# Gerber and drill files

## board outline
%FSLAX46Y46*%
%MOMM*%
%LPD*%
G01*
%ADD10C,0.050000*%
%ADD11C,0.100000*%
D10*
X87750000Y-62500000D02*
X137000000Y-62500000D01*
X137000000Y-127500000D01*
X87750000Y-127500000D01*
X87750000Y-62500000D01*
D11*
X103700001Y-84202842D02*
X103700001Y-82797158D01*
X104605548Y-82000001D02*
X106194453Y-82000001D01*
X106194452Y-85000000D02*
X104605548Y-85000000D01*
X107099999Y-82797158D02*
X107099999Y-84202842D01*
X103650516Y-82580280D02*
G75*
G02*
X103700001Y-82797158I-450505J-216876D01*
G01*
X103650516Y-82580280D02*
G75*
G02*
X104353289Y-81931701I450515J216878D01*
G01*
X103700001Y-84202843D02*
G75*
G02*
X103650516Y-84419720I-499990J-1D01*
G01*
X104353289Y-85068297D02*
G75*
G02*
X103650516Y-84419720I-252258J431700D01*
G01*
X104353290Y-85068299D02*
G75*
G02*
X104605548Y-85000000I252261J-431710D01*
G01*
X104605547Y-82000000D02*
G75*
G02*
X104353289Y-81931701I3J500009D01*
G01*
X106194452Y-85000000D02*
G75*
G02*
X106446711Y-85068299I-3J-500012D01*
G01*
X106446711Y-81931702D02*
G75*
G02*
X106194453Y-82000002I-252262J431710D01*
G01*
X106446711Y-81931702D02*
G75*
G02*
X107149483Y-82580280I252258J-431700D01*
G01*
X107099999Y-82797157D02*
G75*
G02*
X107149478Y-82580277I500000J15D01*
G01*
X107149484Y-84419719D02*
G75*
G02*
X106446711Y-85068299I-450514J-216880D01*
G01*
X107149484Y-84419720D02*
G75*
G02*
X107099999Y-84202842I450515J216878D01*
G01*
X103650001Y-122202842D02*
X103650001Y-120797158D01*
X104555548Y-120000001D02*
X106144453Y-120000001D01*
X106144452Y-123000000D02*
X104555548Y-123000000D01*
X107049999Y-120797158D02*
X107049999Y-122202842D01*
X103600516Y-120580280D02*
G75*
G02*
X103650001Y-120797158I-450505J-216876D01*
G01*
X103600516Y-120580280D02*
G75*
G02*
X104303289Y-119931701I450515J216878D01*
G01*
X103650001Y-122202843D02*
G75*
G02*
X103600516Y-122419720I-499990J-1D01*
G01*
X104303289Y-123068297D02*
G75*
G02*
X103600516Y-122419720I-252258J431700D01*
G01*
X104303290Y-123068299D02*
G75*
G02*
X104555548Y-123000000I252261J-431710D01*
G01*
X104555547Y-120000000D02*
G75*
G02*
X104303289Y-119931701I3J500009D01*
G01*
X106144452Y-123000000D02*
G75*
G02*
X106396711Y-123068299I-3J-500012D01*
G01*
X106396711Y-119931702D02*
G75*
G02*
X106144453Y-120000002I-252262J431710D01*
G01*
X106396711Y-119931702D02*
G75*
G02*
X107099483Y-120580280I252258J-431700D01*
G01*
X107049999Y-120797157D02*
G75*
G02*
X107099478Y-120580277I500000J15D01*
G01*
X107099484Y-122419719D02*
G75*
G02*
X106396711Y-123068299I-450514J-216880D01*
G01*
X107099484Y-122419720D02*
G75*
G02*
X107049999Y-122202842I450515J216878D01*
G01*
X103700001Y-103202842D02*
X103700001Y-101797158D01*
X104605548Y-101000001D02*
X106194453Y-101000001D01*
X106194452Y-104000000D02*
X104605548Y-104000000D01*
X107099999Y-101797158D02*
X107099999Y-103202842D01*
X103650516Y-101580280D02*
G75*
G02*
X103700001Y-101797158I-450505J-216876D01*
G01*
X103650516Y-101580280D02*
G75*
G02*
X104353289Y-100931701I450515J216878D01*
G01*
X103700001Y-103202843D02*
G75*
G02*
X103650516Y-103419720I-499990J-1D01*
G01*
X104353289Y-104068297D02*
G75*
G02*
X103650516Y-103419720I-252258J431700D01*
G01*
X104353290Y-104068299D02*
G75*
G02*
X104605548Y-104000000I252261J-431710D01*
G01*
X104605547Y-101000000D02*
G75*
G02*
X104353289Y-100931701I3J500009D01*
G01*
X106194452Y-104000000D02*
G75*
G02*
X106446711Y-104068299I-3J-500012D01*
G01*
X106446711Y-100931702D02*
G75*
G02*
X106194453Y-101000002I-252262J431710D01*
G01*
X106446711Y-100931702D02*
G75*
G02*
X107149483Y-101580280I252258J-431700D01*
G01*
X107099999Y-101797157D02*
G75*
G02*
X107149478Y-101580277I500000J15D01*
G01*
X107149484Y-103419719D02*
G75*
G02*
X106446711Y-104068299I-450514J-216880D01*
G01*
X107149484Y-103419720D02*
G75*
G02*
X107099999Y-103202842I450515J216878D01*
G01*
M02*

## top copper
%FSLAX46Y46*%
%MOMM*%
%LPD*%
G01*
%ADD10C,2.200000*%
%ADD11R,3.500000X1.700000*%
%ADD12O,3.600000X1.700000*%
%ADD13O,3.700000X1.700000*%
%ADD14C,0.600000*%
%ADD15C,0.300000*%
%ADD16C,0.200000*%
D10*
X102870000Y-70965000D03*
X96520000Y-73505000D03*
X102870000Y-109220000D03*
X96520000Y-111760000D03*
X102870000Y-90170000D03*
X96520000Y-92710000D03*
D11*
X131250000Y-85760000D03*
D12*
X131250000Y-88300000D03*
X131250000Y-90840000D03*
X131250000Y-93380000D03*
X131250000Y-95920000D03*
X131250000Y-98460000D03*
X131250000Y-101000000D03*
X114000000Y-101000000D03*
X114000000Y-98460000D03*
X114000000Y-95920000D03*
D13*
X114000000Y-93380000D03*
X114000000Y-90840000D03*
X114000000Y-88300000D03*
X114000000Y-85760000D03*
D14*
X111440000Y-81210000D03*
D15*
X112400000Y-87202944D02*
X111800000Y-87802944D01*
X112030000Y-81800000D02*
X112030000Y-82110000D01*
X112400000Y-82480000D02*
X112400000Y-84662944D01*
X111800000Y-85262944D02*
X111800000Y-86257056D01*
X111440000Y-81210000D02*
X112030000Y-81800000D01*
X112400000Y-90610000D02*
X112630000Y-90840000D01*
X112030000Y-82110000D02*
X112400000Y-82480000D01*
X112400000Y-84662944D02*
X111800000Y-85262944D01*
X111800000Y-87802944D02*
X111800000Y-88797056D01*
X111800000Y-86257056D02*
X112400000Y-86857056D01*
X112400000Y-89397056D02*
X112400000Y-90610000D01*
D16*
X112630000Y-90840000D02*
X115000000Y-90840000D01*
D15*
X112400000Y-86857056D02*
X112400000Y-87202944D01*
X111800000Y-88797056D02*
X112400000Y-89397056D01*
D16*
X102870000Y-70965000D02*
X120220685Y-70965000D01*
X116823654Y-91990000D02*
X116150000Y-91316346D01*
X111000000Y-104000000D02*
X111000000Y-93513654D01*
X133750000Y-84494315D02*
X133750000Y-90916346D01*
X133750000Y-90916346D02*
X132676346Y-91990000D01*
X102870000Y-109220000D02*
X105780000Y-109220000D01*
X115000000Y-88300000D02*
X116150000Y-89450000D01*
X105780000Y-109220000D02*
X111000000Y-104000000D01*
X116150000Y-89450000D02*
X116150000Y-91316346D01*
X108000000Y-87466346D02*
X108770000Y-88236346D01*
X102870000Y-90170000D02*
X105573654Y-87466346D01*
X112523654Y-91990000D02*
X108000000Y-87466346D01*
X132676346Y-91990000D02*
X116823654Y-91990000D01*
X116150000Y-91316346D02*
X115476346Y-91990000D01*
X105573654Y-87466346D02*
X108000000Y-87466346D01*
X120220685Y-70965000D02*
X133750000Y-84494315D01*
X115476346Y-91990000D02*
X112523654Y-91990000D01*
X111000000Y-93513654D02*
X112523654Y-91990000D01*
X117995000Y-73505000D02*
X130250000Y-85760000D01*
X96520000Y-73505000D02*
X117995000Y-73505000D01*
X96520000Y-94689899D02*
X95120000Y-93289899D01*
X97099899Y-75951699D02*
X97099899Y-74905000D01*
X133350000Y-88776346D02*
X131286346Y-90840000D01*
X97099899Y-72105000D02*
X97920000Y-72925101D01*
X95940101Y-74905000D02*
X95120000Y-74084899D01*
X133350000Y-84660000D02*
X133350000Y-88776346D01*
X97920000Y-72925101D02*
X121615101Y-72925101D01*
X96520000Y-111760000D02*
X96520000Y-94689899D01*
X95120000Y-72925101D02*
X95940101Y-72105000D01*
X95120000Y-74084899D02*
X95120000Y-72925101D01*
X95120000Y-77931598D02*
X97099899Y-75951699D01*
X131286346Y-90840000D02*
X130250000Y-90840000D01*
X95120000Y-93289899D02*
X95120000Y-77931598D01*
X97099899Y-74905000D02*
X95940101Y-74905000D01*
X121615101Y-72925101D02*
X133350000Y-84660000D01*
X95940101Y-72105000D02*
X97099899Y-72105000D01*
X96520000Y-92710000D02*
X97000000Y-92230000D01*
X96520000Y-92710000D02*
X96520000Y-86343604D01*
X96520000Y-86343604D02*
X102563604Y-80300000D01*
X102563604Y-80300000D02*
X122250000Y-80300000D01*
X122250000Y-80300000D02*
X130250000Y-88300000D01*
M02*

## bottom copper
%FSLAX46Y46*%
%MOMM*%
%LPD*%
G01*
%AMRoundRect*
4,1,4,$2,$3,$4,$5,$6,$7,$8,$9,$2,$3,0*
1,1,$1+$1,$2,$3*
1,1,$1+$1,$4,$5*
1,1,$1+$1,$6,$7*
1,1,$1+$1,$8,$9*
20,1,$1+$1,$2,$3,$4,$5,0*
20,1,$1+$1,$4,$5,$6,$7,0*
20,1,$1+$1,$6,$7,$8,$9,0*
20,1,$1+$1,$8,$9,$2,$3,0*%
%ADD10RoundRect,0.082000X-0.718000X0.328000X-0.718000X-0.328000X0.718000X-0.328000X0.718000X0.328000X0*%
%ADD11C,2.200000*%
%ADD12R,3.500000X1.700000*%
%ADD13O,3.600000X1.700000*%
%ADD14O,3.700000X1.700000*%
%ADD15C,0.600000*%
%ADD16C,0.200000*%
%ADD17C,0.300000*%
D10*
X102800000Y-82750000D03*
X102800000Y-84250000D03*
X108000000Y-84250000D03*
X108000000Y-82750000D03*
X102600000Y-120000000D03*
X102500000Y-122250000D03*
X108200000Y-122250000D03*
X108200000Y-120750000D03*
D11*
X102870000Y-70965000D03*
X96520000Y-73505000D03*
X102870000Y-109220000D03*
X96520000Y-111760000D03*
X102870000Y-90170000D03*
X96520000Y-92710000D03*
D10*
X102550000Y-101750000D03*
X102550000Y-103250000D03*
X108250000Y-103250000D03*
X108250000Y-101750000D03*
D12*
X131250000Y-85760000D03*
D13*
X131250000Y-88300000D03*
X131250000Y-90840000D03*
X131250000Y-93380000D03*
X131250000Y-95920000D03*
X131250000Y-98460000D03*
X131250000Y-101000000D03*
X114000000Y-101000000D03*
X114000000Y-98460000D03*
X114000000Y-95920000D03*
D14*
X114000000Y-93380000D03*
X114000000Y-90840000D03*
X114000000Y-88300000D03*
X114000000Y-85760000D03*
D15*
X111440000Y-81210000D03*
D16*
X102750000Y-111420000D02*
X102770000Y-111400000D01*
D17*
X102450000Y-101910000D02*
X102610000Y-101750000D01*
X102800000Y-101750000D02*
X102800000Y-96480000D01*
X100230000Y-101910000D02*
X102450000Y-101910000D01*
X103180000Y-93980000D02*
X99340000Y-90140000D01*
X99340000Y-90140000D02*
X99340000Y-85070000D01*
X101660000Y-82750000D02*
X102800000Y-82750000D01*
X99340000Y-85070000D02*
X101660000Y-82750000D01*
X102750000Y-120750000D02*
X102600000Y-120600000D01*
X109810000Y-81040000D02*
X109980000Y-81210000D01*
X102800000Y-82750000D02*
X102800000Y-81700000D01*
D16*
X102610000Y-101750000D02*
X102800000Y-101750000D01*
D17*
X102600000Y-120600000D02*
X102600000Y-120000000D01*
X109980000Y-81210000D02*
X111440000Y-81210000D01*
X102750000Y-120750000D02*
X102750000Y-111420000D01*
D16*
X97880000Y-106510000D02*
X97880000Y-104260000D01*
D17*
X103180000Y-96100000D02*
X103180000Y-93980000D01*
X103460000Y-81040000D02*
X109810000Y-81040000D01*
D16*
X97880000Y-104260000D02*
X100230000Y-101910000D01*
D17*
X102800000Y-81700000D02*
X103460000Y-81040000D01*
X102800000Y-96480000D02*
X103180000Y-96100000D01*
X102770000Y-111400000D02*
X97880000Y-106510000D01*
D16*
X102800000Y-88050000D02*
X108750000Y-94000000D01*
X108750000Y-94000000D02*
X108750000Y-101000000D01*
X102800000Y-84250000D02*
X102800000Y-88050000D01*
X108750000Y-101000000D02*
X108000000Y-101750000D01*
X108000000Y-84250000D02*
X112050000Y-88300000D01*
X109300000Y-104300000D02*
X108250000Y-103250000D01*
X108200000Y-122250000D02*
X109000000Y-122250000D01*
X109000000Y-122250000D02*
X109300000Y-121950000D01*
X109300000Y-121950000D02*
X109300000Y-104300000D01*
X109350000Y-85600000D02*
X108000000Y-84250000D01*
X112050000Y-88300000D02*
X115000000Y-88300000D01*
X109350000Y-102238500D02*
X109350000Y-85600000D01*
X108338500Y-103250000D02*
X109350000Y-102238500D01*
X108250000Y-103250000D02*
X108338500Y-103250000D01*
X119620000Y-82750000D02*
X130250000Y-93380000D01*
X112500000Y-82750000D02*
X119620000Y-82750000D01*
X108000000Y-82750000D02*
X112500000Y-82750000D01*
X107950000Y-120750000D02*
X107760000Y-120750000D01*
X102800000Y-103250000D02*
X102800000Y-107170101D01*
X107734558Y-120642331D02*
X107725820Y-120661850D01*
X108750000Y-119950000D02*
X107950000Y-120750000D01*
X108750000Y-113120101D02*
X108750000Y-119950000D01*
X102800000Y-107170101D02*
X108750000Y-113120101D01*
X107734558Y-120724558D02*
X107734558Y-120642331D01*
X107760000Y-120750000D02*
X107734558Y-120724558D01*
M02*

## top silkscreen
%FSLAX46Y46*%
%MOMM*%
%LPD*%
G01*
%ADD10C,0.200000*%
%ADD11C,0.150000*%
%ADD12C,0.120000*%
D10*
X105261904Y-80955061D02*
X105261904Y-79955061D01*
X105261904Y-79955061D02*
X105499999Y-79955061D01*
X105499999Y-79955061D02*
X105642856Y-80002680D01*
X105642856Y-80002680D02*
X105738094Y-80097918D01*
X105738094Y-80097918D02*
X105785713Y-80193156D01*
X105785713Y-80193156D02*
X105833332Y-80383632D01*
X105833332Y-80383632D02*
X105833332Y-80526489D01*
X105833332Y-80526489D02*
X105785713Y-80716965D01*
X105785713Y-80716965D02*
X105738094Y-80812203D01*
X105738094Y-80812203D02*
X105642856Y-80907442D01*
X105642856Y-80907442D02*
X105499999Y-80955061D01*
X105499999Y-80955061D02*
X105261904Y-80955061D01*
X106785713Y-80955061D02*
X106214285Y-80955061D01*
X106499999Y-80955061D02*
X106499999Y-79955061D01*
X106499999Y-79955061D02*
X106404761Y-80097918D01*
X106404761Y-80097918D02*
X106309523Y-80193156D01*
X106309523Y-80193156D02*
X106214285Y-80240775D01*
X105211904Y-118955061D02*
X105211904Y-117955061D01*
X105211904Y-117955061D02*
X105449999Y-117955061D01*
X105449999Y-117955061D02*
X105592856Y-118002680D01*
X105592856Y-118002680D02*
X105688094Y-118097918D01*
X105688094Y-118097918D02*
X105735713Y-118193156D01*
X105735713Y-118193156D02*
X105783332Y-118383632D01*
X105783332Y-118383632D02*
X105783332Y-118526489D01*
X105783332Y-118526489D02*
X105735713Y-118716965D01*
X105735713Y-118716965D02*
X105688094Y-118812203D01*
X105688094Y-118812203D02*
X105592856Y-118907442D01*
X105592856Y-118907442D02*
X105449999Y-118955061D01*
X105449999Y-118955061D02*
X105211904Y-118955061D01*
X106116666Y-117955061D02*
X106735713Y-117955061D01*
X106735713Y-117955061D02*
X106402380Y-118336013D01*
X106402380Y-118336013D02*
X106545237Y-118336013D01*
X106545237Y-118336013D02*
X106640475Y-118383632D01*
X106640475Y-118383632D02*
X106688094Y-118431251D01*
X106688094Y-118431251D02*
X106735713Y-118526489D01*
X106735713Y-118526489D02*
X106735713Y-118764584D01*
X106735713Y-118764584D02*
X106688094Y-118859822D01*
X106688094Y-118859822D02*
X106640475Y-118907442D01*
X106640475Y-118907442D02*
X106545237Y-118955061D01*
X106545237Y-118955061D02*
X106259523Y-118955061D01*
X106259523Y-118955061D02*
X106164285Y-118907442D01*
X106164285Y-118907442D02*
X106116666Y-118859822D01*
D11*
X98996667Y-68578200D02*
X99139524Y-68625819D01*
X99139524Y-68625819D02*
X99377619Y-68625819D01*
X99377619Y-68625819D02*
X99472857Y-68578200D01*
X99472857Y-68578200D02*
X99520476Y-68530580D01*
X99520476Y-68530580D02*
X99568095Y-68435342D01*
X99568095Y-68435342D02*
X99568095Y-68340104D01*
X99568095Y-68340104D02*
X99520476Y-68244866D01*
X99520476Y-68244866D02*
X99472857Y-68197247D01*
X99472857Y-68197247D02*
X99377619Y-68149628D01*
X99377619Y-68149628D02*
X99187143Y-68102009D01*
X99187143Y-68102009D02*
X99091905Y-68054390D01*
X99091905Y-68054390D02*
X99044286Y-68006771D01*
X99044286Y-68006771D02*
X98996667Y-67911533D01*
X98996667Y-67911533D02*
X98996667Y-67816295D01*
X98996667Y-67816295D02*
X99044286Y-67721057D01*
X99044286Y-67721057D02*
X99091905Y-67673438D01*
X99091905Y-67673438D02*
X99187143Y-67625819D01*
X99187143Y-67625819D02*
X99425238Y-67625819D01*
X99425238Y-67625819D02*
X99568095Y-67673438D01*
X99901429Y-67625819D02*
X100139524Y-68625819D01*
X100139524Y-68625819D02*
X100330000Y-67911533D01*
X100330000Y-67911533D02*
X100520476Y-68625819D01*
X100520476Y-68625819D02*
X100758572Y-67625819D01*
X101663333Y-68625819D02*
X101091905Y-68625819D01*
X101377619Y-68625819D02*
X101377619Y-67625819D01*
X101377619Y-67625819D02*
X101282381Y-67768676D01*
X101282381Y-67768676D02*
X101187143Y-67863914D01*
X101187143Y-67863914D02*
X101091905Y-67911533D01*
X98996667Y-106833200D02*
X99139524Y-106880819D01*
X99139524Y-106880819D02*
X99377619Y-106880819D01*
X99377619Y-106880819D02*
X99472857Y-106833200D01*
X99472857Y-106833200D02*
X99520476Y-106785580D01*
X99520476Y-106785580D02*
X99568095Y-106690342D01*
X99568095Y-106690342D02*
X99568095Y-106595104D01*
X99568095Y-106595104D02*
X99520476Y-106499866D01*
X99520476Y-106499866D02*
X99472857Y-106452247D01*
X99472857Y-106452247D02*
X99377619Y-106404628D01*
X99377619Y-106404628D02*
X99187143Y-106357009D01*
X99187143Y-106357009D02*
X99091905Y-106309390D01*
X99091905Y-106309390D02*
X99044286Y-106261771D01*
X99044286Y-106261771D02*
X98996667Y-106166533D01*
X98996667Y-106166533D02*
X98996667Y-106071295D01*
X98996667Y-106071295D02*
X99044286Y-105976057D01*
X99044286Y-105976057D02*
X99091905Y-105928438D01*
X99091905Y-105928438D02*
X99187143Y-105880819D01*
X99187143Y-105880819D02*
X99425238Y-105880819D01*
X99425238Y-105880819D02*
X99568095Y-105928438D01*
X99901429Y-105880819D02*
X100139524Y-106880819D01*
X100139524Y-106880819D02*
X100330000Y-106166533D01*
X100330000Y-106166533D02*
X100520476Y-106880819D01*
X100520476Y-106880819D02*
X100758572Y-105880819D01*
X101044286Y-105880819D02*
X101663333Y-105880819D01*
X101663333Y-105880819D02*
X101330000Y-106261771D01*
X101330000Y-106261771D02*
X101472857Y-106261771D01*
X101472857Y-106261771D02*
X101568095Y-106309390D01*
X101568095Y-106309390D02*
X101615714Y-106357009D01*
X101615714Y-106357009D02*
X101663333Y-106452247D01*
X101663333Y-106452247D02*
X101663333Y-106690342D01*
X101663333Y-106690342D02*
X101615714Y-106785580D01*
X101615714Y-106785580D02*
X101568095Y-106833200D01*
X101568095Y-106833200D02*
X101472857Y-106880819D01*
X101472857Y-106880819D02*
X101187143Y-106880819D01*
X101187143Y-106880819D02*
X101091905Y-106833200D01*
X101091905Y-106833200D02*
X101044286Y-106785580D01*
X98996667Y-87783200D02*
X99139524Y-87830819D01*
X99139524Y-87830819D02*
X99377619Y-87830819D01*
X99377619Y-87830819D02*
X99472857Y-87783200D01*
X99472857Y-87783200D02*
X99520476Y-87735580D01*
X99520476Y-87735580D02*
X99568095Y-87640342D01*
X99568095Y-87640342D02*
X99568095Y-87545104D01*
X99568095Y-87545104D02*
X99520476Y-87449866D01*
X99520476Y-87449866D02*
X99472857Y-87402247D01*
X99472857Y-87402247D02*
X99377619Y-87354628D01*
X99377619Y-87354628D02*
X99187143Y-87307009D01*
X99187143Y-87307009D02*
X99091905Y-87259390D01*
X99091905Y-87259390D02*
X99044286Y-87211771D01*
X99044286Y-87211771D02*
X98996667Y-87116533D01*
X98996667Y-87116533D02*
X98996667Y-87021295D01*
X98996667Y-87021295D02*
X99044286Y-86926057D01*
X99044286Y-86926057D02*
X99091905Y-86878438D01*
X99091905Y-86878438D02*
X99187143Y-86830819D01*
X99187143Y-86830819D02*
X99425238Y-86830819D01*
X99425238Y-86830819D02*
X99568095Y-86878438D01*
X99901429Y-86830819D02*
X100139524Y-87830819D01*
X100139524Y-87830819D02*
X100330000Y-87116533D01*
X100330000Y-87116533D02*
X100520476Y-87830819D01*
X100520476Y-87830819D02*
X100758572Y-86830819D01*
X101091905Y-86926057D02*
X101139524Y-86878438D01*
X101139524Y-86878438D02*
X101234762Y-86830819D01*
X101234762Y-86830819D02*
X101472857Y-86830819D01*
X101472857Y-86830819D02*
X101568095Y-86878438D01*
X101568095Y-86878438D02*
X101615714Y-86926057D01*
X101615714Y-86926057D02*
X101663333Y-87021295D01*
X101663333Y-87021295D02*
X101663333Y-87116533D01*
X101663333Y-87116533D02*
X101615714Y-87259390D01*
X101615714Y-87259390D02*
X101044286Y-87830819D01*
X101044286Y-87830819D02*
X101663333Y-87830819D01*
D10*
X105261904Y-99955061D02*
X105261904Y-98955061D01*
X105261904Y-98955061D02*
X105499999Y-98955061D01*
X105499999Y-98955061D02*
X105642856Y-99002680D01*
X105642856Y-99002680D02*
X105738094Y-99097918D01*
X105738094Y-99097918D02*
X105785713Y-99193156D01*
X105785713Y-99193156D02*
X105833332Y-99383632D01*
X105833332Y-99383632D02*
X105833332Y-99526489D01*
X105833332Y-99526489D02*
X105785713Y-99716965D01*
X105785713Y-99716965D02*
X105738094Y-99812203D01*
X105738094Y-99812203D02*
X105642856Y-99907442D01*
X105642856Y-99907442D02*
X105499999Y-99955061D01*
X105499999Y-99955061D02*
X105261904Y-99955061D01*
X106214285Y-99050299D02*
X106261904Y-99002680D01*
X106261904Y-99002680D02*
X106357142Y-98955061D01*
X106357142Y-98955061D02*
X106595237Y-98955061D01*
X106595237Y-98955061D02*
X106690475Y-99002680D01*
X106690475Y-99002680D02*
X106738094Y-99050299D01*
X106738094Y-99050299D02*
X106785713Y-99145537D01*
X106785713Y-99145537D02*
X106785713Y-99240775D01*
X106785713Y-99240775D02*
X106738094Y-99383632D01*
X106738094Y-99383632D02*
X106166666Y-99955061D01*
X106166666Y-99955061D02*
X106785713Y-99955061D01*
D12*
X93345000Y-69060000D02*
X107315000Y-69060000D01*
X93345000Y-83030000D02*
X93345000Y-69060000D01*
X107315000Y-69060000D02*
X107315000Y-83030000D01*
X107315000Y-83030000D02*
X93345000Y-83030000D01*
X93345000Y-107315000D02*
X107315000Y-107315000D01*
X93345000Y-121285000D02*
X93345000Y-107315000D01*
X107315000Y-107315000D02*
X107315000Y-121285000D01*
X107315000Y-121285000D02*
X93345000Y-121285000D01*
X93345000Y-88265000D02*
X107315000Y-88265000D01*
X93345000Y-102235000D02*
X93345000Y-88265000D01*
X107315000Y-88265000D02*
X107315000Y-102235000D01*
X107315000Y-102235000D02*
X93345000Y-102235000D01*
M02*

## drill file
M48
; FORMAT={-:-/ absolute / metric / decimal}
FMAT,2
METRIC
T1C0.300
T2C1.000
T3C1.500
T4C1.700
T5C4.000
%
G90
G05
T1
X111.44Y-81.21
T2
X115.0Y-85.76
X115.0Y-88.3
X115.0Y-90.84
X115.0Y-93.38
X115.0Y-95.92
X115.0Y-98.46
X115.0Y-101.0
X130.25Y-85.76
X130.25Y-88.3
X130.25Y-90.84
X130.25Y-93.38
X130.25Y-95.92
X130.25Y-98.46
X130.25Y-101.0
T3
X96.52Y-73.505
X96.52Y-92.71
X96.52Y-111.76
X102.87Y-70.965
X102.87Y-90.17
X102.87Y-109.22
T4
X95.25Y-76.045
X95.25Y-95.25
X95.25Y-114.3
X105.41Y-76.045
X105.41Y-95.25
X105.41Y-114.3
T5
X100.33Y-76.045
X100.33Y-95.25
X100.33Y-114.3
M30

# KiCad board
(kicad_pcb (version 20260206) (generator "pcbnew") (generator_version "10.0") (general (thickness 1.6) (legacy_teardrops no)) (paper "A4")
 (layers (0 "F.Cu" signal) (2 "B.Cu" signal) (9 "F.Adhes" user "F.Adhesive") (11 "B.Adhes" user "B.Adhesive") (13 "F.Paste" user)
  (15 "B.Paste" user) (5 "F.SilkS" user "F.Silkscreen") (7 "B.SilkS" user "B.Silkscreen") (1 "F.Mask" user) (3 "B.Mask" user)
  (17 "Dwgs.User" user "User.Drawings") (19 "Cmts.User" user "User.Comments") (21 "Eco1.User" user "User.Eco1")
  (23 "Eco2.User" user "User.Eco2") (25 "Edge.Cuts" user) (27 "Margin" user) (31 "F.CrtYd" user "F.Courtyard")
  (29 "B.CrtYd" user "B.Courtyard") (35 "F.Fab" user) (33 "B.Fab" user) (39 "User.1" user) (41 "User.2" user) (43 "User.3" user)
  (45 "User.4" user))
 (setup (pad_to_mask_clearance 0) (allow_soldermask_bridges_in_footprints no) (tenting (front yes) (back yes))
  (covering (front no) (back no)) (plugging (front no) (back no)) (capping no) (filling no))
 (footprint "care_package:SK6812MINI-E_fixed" (layer "F.Cu") (at 105.399999 83.602842)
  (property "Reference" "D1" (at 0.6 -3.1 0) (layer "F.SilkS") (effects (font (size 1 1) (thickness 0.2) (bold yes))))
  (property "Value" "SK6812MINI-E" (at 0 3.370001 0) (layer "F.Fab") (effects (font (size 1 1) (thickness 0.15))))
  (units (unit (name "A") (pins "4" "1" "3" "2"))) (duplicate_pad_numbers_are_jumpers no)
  (fp_line (start -1.699998 0.6) (end -1.699998 -0.805684) (stroke (width 0.1) (type solid)) (layer "Edge.Cuts"))
  (fp_line (start -0.794451 -1.602841) (end 0.794454 -1.602841) (stroke (width 0.1) (type solid)) (layer "Edge.Cuts"))
  (fp_line (start 0.794453 1.397158) (end -0.794451 1.397158) (stroke (width 0.1) (type solid)) (layer "Edge.Cuts"))
  (fp_line (start 1.7 -0.805684) (end 1.7 0.6) (stroke (width 0.1) (type solid)) (layer "Edge.Cuts"))
  (fp_arc (start -1.749483 -1.022562) (mid -1.712526 -0.91691) (end -1.699998 -0.805684) (stroke (width 0.1) (type solid))
   (layer "Edge.Cuts"))
  (fp_arc (start -1.749483 -1.022562) (mid -1.63807 -1.606877) (end -1.04671 -1.671141) (stroke (width 0.1) (type solid))
   (layer "Edge.Cuts"))
  (fp_arc (start -1.699998 0.600001) (mid -1.712526 0.711226) (end -1.749483 0.816878) (stroke (width 0.1) (type solid)) (layer "Edge.Cuts"))
  (fp_arc (start -1.04671 1.465455) (mid -1.638069 1.401192) (end -1.749483 0.816878) (stroke (width 0.1) (type solid)) (layer "Edge.Cuts"))
  (fp_arc (start -1.046709 1.465457) (mid -0.925121 1.414535) (end -0.794451 1.397158) (stroke (width 0.1) (type solid)) (layer "Edge.Cuts"))
  (fp_arc (start -0.794452 -1.602842) (mid -0.925122 -1.620219) (end -1.04671 -1.671141) (stroke (width 0.1) (type solid))
   (layer "Edge.Cuts"))
  (fp_arc (start 0.794453 1.397158) (mid 0.925124 1.414535) (end 1.046712 1.465457) (stroke (width 0.1) (type solid)) (layer "Edge.Cuts"))
  (fp_arc (start 1.046712 -1.67114) (mid 0.925124 -1.620218) (end 0.794454 -1.602841) (stroke (width 0.1) (type solid)) (layer "Edge.Cuts"))
  (fp_arc (start 1.046712 -1.67114) (mid 1.638072 -1.606876) (end 1.749485 -1.022562) (stroke (width 0.1) (type solid)) (layer "Edge.Cuts"))
  (fp_arc (start 1.7 -0.805685) (mid 1.712528 -0.91691) (end 1.749485 -1.022562) (stroke (width 0.1) (type solid)) (layer "Edge.Cuts"))
  (fp_arc (start 1.749485 0.816877) (mid 1.638073 1.401193) (end 1.046712 1.465457) (stroke (width 0.1) (type solid)) (layer "Edge.Cuts"))
  (fp_arc (start 1.749485 0.816878) (mid 1.712528 0.711226) (end 1.7 0.6) (stroke (width 0.1) (type solid)) (layer "Edge.Cuts"))
  (pad "1" smd roundrect (at -2.599999 -0.852842 270) (size 0.82 1.6) (layers "B.Cu" "B.Mask" "B.Paste") (roundrect_rratio 0.1) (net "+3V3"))
  (pad "2" smd roundrect (at -2.599999 0.647158 270) (size 0.82 1.6) (layers "B.Cu" "B.Mask" "B.Paste") (roundrect_rratio 0.1)
   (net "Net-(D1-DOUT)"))
  (pad "3" smd roundrect (at 2.600001 0.647158 270) (size 0.82 1.6) (layers "B.Cu" "B.Mask" "B.Paste") (roundrect_rratio 0.1) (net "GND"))
  (pad "4" smd roundrect (at 2.600001 -0.852842 270) (size 0.82 1.6) (layers "B.Cu" "B.Mask" "B.Paste") (roundrect_rratio 0.1)
   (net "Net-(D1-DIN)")))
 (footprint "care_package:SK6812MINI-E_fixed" (layer "F.Cu") (at 105.349999 121.602842)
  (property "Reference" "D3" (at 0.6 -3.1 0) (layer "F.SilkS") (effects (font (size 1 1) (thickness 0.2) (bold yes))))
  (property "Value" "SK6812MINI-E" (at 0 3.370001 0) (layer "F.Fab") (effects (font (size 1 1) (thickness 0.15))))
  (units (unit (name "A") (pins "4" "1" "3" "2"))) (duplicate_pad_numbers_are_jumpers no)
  (fp_line (start -1.699998 0.6) (end -1.699998 -0.805684) (stroke (width 0.1) (type solid)) (layer "Edge.Cuts"))
  (fp_line (start -0.794451 -1.602841) (end 0.794454 -1.602841) (stroke (width 0.1) (type solid)) (layer "Edge.Cuts"))
  (fp_line (start 0.794453 1.397158) (end -0.794451 1.397158) (stroke (width 0.1) (type solid)) (layer "Edge.Cuts"))
  (fp_line (start 1.7 -0.805684) (end 1.7 0.6) (stroke (width 0.1) (type solid)) (layer "Edge.Cuts"))
  (fp_arc (start -1.749483 -1.022562) (mid -1.712526 -0.91691) (end -1.699998 -0.805684) (stroke (width 0.1) (type solid))
   (layer "Edge.Cuts"))
  (fp_arc (start -1.749483 -1.022562) (mid -1.63807 -1.606877) (end -1.04671 -1.671141) (stroke (width 0.1) (type solid))
   (layer "Edge.Cuts"))
  (fp_arc (start -1.699998 0.600001) (mid -1.712526 0.711226) (end -1.749483 0.816878) (stroke (width 0.1) (type solid)) (layer "Edge.Cuts"))
  (fp_arc (start -1.04671 1.465455) (mid -1.638069 1.401192) (end -1.749483 0.816878) (stroke (width 0.1) (type solid)) (layer "Edge.Cuts"))
  (fp_arc (start -1.046709 1.465457) (mid -0.925121 1.414535) (end -0.794451 1.397158) (stroke (width 0.1) (type solid)) (layer "Edge.Cuts"))
  (fp_arc (start -0.794452 -1.602842) (mid -0.925122 -1.620219) (end -1.04671 -1.671141) (stroke (width 0.1) (type solid))
   (layer "Edge.Cuts"))
  (fp_arc (start 0.794453 1.397158) (mid 0.925124 1.414535) (end 1.046712 1.465457) (stroke (width 0.1) (type solid)) (layer "Edge.Cuts"))
  (fp_arc (start 1.046712 -1.67114) (mid 0.925124 -1.620218) (end 0.794454 -1.602841) (stroke (width 0.1) (type solid)) (layer "Edge.Cuts"))
  (fp_arc (start 1.046712 -1.67114) (mid 1.638072 -1.606876) (end 1.749485 -1.022562) (stroke (width 0.1) (type solid)) (layer "Edge.Cuts"))
  (fp_arc (start 1.7 -0.805685) (mid 1.712528 -0.91691) (end 1.749485 -1.022562) (stroke (width 0.1) (type solid)) (layer "Edge.Cuts"))
  (fp_arc (start 1.749485 0.816877) (mid 1.638073 1.401193) (end 1.046712 1.465457) (stroke (width 0.1) (type solid)) (layer "Edge.Cuts"))
  (fp_arc (start 1.749485 0.816878) (mid 1.712528 0.711226) (end 1.7 0.6) (stroke (width 0.1) (type solid)) (layer "Edge.Cuts"))
  (pad "1" smd roundrect (at -2.749999 -1.602842 270) (size 0.82 1.6) (layers "B.Cu" "B.Mask" "B.Paste") (roundrect_rratio 0.1) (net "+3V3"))
  (pad "2" smd roundrect (at -2.849999 0.647158 270) (size 0.82 1.6) (layers "B.Cu" "B.Mask" "B.Paste") (roundrect_rratio 0.1)
   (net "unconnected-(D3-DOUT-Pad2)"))
  (pad "3" smd roundrect (at 2.850001 0.647158 270) (size 0.82 1.6) (layers "B.Cu" "B.Mask" "B.Paste") (roundrect_rratio 0.1) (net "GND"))
  (pad "4" smd roundrect (at 2.850001 -0.852842 270) (size 0.82 1.6) (layers "B.Cu" "B.Mask" "B.Paste") (roundrect_rratio 0.1)
   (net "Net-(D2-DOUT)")))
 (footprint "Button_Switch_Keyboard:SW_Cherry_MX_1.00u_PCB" (layer "F.Cu") (at 102.87 70.965)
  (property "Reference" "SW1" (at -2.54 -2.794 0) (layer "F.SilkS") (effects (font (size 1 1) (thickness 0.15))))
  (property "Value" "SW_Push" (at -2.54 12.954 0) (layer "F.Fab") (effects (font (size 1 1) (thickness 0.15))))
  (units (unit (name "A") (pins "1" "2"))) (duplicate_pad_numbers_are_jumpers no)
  (fp_line (start -9.525 -1.905) (end 4.445 -1.905) (stroke (width 0.12) (type solid)) (layer "F.SilkS"))
  (fp_line (start -9.525 12.065) (end -9.525 -1.905) (stroke (width 0.12) (type solid)) (layer "F.SilkS"))
  (fp_line (start 4.445 -1.905) (end 4.445 12.065) (stroke (width 0.12) (type solid)) (layer "F.SilkS"))
  (fp_line (start 4.445 12.065) (end -9.525 12.065) (stroke (width 0.12) (type solid)) (layer "F.SilkS"))
  (pad "" np_thru_hole circle (at -7.62 5.08) (size 1.7 1.7) (drill 1.7) (layers "*.Cu" "*.Mask"))
  (pad "" np_thru_hole circle (at -2.54 5.08) (size 4 4) (drill 4) (layers "*.Cu" "*.Mask"))
  (pad "" np_thru_hole circle (at 2.54 5.08) (size 1.7 1.7) (drill 1.7) (layers "*.Cu" "*.Mask"))
  (pad "1" thru_hole circle (at 0 0) (size 2.2 2.2) (drill 1.5) (layers "*.Cu" "*.Mask") (remove_unused_layers no) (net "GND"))
  (pad "2" thru_hole circle (at -6.35 2.54) (size 2.2 2.2) (drill 1.5) (layers "*.Cu" "*.Mask") (remove_unused_layers no)
   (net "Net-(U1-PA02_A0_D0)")))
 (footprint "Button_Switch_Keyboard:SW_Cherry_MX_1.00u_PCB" (layer "F.Cu") (at 102.87 109.22)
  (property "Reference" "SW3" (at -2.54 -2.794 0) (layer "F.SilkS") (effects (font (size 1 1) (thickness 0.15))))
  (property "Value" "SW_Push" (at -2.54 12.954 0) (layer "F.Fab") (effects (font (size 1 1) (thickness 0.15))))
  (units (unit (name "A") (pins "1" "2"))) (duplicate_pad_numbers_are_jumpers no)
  (fp_line (start -9.525 -1.905) (end 4.445 -1.905) (stroke (width 0.12) (type solid)) (layer "F.SilkS"))
  (fp_line (start -9.525 12.065) (end -9.525 -1.905) (stroke (width 0.12) (type solid)) (layer "F.SilkS"))
  (fp_line (start 4.445 -1.905) (end 4.445 12.065) (stroke (width 0.12) (type solid)) (layer "F.SilkS"))
  (fp_line (start 4.445 12.065) (end -9.525 12.065) (stroke (width 0.12) (type solid)) (layer "F.SilkS"))
  (pad "" np_thru_hole circle (at -7.62 5.08) (size 1.7 1.7) (drill 1.7) (layers "*.Cu" "*.Mask"))
  (pad "" np_thru_hole circle (at -2.54 5.08) (size 4 4) (drill 4) (layers "*.Cu" "*.Mask"))
  (pad "" np_thru_hole circle (at 2.54 5.08) (size 1.7 1.7) (drill 1.7) (layers "*.Cu" "*.Mask"))
  (pad "1" thru_hole circle (at 0 0) (size 2.2 2.2) (drill 1.5) (layers "*.Cu" "*.Mask") (remove_unused_layers no) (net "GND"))
  (pad "2" thru_hole circle (at -6.35 2.54) (size 2.2 2.2) (drill 1.5) (layers "*.Cu" "*.Mask") (remove_unused_layers no)
   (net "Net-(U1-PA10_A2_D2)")))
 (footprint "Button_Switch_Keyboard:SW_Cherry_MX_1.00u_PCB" (layer "F.Cu") (at 102.87 90.17)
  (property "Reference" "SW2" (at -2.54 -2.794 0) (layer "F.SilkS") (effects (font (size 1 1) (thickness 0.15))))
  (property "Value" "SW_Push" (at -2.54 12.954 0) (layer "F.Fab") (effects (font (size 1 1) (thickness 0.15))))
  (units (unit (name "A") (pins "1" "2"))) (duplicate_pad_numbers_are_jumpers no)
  (fp_line (start -9.525 -1.905) (end 4.445 -1.905) (stroke (width 0.12) (type solid)) (layer "F.SilkS"))
  (fp_line (start -9.525 12.065) (end -9.525 -1.905) (stroke (width 0.12) (type solid)) (layer "F.SilkS"))
  (fp_line (start 4.445 -1.905) (end 4.445 12.065) (stroke (width 0.12) (type solid)) (layer "F.SilkS"))
  (fp_line (start 4.445 12.065) (end -9.525 12.065) (stroke (width 0.12) (type solid)) (layer "F.SilkS"))
  (pad "" np_thru_hole circle (at -7.62 5.08) (size 1.7 1.7) (drill 1.7) (layers "*.Cu" "*.Mask"))
  (pad "" np_thru_hole circle (at -2.54 5.08) (size 4 4) (drill 4) (layers "*.Cu" "*.Mask"))
  (pad "" np_thru_hole circle (at 2.54 5.08) (size 1.7 1.7) (drill 1.7) (layers "*.Cu" "*.Mask"))
  (pad "1" thru_hole circle (at 0 0) (size 2.2 2.2) (drill 1.5) (layers "*.Cu" "*.Mask") (remove_unused_layers no) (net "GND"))
  (pad "2" thru_hole circle (at -6.35 2.54) (size 2.2 2.2) (drill 1.5) (layers "*.Cu" "*.Mask") (remove_unused_layers no)
   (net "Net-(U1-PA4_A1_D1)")))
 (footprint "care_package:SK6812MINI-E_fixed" (layer "F.Cu") (at 105.399999 102.602842)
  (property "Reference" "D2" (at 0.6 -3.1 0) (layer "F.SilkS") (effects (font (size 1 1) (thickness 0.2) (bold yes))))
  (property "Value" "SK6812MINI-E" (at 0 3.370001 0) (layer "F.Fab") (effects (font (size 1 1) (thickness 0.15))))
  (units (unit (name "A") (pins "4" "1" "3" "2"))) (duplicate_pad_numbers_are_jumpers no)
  (fp_line (start -1.699998 0.6) (end -1.699998 -0.805684) (stroke (width 0.1) (type solid)) (layer "Edge.Cuts"))
  (fp_line (start -0.794451 -1.602841) (end 0.794454 -1.602841) (stroke (width 0.1) (type solid)) (layer "Edge.Cuts"))
  (fp_line (start 0.794453 1.397158) (end -0.794451 1.397158) (stroke (width 0.1) (type solid)) (layer "Edge.Cuts"))
  (fp_line (start 1.7 -0.805684) (end 1.7 0.6) (stroke (width 0.1) (type solid)) (layer "Edge.Cuts"))
  (fp_arc (start -1.749483 -1.022562) (mid -1.712526 -0.91691) (end -1.699998 -0.805684) (stroke (width 0.1) (type solid))
   (layer "Edge.Cuts"))
  (fp_arc (start -1.749483 -1.022562) (mid -1.63807 -1.606877) (end -1.04671 -1.671141) (stroke (width 0.1) (type solid))
   (layer "Edge.Cuts"))
  (fp_arc (start -1.699998 0.600001) (mid -1.712526 0.711226) (end -1.749483 0.816878) (stroke (width 0.1) (type solid)) (layer "Edge.Cuts"))
  (fp_arc (start -1.04671 1.465455) (mid -1.638069 1.401192) (end -1.749483 0.816878) (stroke (width 0.1) (type solid)) (layer "Edge.Cuts"))
  (fp_arc (start -1.046709 1.465457) (mid -0.925121 1.414535) (end -0.794451 1.397158) (stroke (width 0.1) (type solid)) (layer "Edge.Cuts"))
  (fp_arc (start -0.794452 -1.602842) (mid -0.925122 -1.620219) (end -1.04671 -1.671141) (stroke (width 0.1) (type solid))
   (layer "Edge.Cuts"))
  (fp_arc (start 0.794453 1.397158) (mid 0.925124 1.414535) (end 1.046712 1.465457) (stroke (width 0.1) (type solid)) (layer "Edge.Cuts"))
  (fp_arc (start 1.046712 -1.67114) (mid 0.925124 -1.620218) (end 0.794454 -1.602841) (stroke (width 0.1) (type solid)) (layer "Edge.Cuts"))
  (fp_arc (start 1.046712 -1.67114) (mid 1.638072 -1.606876) (end 1.749485 -1.022562) (stroke (width 0.1) (type solid)) (layer "Edge.Cuts"))
  (fp_arc (start 1.7 -0.805685) (mid 1.712528 -0.91691) (end 1.749485 -1.022562) (stroke (width 0.1) (type solid)) (layer "Edge.Cuts"))
  (fp_arc (start 1.749485 0.816877) (mid 1.638073 1.401193) (end 1.046712 1.465457) (stroke (width 0.1) (type solid)) (layer "Edge.Cuts"))
  (fp_arc (start 1.749485 0.816878) (mid 1.712528 0.711226) (end 1.7 0.6) (stroke (width 0.1) (type solid)) (layer "Edge.Cuts"))
  (pad "1" smd roundrect (at -2.849999 -0.852842 270) (size 0.82 1.6) (layers "B.Cu" "B.Mask" "B.Paste") (roundrect_rratio 0.1) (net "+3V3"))
  (pad "2" smd roundrect (at -2.849999 0.647158 270) (size 0.82 1.6) (layers "B.Cu" "B.Mask" "B.Paste") (roundrect_rratio 0.1)
   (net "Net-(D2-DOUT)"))
  (pad "3" smd roundrect (at 2.850001 0.647158 270) (size 0.82 1.6) (layers "B.Cu" "B.Mask" "B.Paste") (roundrect_rratio 0.1) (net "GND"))
  (pad "4" smd roundrect (at 2.850001 -0.852842 270) (size 0.82 1.6) (layers "B.Cu" "B.Mask" "B.Paste") (roundrect_rratio 0.1)
   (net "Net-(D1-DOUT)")))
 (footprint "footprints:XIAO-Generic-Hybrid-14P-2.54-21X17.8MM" (layer "B.Cu") (at 122.625 93.38 180)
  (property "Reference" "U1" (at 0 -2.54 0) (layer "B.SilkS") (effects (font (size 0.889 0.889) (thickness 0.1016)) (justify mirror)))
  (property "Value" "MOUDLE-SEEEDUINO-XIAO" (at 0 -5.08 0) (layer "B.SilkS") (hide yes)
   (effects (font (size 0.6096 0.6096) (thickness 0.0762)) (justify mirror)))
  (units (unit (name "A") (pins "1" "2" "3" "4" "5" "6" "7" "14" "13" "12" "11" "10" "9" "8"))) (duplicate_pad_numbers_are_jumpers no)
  (pad "1" thru_hole rect (at -7.625 7.62 180) (size 3.5 1.7) (drill 1 (offset -1 0)) (layers "*.Cu" "*.Mask") (remove_unused_layers no)
   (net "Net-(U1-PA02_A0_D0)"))
  (pad "2" thru_hole oval (at -7.625 5.08 180) (size 3.6 1.7) (drill 1 (offset -1 0)) (layers "*.Cu" "*.Mask") (remove_unused_layers no)
   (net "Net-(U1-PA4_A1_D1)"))
  (pad "3" thru_hole oval (at -7.625 2.54 180) (size 3.6 1.7) (drill 1 (offset -1 0)) (layers "*.Cu" "*.Mask") (remove_unused_layers no)
   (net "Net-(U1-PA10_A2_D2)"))
  (pad "4" thru_hole oval (at -7.625 0 180) (size 3.6 1.7) (drill 1 (offset -1 0)) (layers "*.Cu" "*.Mask") (remove_unused_layers no)
   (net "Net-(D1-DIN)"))
  (pad "5" thru_hole oval (at -7.625 -2.54 180) (size 3.6 1.7) (drill 1 (offset -1 0)) (layers "*.Cu" "*.Mask") (remove_unused_layers no)
   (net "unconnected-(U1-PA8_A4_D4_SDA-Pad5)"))
  (pad "6" thru_hole oval (at -7.625 -5.08) (size 3.6 1.7) (drill 1 (offset 1 0)) (layers "*.Cu" "*.Mask") (remove_unused_layers no)
   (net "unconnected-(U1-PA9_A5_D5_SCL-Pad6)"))
  (pad "7" thru_hole oval (at -7.625 -7.62 180) (size 3.6 1.7) (drill 1 (offset -1 0)) (layers "*.Cu" "*.Mask") (remove_unused_layers no)
   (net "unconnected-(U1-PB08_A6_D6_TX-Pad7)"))
  (pad "8" thru_hole oval (at 7.625 -7.62 180) (size 3.6 1.7) (drill 1 (offset 1 0)) (layers "*.Cu" "*.Mask") (remove_unused_layers no)
   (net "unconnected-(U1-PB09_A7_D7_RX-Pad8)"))
  (pad "9" thru_hole oval (at 7.625 -5.08 180) (size 3.6 1.7) (drill 1 (offset 1 0)) (layers "*.Cu" "*.Mask") (remove_unused_layers no)
   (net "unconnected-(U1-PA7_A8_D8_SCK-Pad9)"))
  (pad "10" thru_hole oval (at 7.625 -2.54 180) (size 3.6 1.7) (drill 1 (offset 1 0)) (layers "*.Cu" "*.Mask") (remove_unused_layers no)
   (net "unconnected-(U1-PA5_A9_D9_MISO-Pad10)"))
  (pad "11" thru_hole oval (at 7.625 0 180) (size 3.7 1.7) (drill 1 (offset 1 0)) (layers "*.Cu" "*.Mask") (remove_unused_layers no)
   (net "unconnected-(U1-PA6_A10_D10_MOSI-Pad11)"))
  (pad "12" thru_hole oval (at 7.625 2.54 180) (size 3.7 1.7) (drill 1 (offset 1 0)) (layers "*.Cu" "*.Mask") (remove_unused_layers no)
   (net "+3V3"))
  (pad "13" thru_hole oval (at 7.625 5.08 180) (size 3.7 1.7) (drill 1 (offset 1 0)) (layers "*.Cu" "*.Mask") (remove_unused_layers no)
   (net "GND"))
  (pad "14" thru_hole oval (at 7.625 7.62 180) (size 3.7 1.7) (drill 1 (offset 1 0)) (layers "*.Cu" "*.Mask") (remove_unused_layers no)
   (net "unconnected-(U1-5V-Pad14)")))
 (gr_rect (start 87.75 62.5) (end 137 127.5) (stroke (width 0.05) (type default)) (fill no) (layer "Edge.Cuts"))
 (segment (start 112.4 87.202944) (end 111.8 87.802944) (width 0.3) (layer "F.Cu") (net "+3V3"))
 (segment (start 112.03 81.8) (end 112.03 82.11) (width 0.3) (layer "F.Cu") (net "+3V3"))
 (segment (start 112.4 82.48) (end 112.4 84.662944) (width 0.3) (layer "F.Cu") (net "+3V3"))
 (segment (start 111.8 85.262944) (end 111.8 86.257056) (width 0.3) (layer "F.Cu") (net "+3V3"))
 (segment (start 111.44 81.21) (end 112.03 81.8) (width 0.3) (layer "F.Cu") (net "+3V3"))
 (segment (start 112.4 90.61) (end 112.63 90.84) (width 0.3) (layer "F.Cu") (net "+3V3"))
 (segment (start 112.03 82.11) (end 112.4 82.48) (width 0.3) (layer "F.Cu") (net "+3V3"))
 (segment (start 112.4 84.662944) (end 111.8 85.262944) (width 0.3) (layer "F.Cu") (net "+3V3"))
 (segment (start 111.8 87.802944) (end 111.8 88.797056) (width 0.3) (layer "F.Cu") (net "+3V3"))
 (segment (start 111.8 86.257056) (end 112.4 86.857056) (width 0.3) (layer "F.Cu") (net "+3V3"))
 (segment (start 112.4 89.397056) (end 112.4 90.61) (width 0.3) (layer "F.Cu") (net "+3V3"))
 (segment (start 112.63 90.84) (end 115 90.84) (width 0.2) (layer "F.Cu") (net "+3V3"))
 (segment (start 112.4 86.857056) (end 112.4 87.202944) (width 0.3) (layer "F.Cu") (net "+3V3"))
 (segment (start 111.8 88.797056) (end 112.4 89.397056) (width 0.3) (layer "F.Cu") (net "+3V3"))
 (via (at 111.44 81.21) (size 0.6) (drill 0.3) (layers "F.Cu" "B.Cu") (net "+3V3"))
 (segment (start 102.75 111.42) (end 102.77 111.4) (width 0.2) (layer "B.Cu") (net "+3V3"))
 (segment (start 102.45 101.91) (end 102.61 101.75) (width 0.3) (layer "B.Cu") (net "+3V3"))
 (segment (start 102.8 101.75) (end 102.8 96.48) (width 0.3) (layer "B.Cu") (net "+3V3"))
 (segment (start 100.23 101.91) (end 102.45 101.91) (width 0.3) (layer "B.Cu") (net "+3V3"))
 (segment (start 103.18 93.98) (end 99.34 90.14) (width 0.3) (layer "B.Cu") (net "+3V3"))
 (segment (start 99.34 90.14) (end 99.34 85.07) (width 0.3) (layer "B.Cu") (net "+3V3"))
 (segment (start 101.66 82.75) (end 102.8 82.75) (width 0.3) (layer "B.Cu") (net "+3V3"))
 (segment (start 99.34 85.07) (end 101.66 82.75) (width 0.3) (layer "B.Cu") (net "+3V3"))
 (segment (start 102.75 120.75) (end 102.6 120.6) (width 0.3) (layer "B.Cu") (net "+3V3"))
 (segment (start 109.81 81.04) (end 109.98 81.21) (width 0.3) (layer "B.Cu") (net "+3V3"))
 (segment (start 102.8 82.75) (end 102.8 81.7) (width 0.3) (layer "B.Cu") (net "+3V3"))
 (segment (start 102.61 101.75) (end 102.8 101.75) (width 0.2) (layer "B.Cu") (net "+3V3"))
 (segment (start 102.6 120.6) (end 102.6 120) (width 0.3) (layer "B.Cu") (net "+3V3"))
 (segment (start 109.98 81.21) (end 111.44 81.21) (width 0.3) (layer "B.Cu") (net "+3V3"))
 (segment (start 102.75 120.75) (end 102.75 111.42) (width 0.3) (layer "B.Cu") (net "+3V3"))
 (segment (start 97.88 106.51) (end 97.88 104.26) (width 0.2) (layer "B.Cu") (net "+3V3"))
 (segment (start 103.18 96.1) (end 103.18 93.98) (width 0.3) (layer "B.Cu") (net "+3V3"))
 (segment (start 103.46 81.04) (end 109.81 81.04) (width 0.3) (layer "B.Cu") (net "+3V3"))
 (segment (start 97.88 104.26) (end 100.23 101.91) (width 0.2) (layer "B.Cu") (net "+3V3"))
 (segment (start 102.8 81.7) (end 103.46 81.04) (width 0.3) (layer "B.Cu") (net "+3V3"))
 (segment (start 102.8 96.48) (end 103.18 96.1) (width 0.3) (layer "B.Cu") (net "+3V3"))
 (segment (start 102.77 111.4) (end 97.88 106.51) (width 0.3) (layer "B.Cu") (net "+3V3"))
 (segment (start 102.8 88.05) (end 108.75 94) (width 0.2) (layer "B.Cu") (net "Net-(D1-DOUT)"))
 (segment (start 108.75 94) (end 108.75 101) (width 0.2) (layer "B.Cu") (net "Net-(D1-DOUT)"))
 (segment (start 102.8 84.25) (end 102.8 88.05) (width 0.2) (layer "B.Cu") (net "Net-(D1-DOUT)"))
 (segment (start 108.75 101) (end 108 101.75) (width 0.2) (layer "B.Cu") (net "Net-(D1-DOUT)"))
 (segment (start 102.87 70.965) (end 120.220685 70.965) (width 0.2) (layer "F.Cu") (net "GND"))
 (segment (start 116.823654 91.99) (end 116.15 91.316346) (width 0.2) (layer "F.Cu") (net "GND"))
 (segment (start 111 104) (end 111 93.513654) (width 0.2) (layer "F.Cu") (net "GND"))
 (segment (start 133.75 84.494315) (end 133.75 90.916346) (width 0.2) (layer "F.Cu") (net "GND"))
 (segment (start 133.75 90.916346) (end 132.676346 91.99) (width 0.2) (layer "F.Cu") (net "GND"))
 (segment (start 102.87 109.22) (end 105.78 109.22) (width 0.2) (layer "F.Cu") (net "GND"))
 (segment (start 115 88.3) (end 116.15 89.45) (width 0.2) (layer "F.Cu") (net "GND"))
 (segment (start 105.78 109.22) (end 111 104) (width 0.2) (layer "F.Cu") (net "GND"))
 (segment (start 116.15 89.45) (end 116.15 91.316346) (width 0.2) (layer "F.Cu") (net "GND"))
 (segment (start 108 87.466346) (end 108.77 88.236346) (width 0.2) (layer "F.Cu") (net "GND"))
 (segment (start 102.87 90.17) (end 105.573654 87.466346) (width 0.2) (layer "F.Cu") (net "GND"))
 (segment (start 112.523654 91.99) (end 108 87.466346) (width 0.2) (layer "F.Cu") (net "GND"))
 (segment (start 132.676346 91.99) (end 116.823654 91.99) (width 0.2) (layer "F.Cu") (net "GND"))
 (segment (start 116.15 91.316346) (end 115.476346 91.99) (width 0.2) (layer "F.Cu") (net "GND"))
 (segment (start 105.573654 87.466346) (end 108 87.466346) (width 0.2) (layer "F.Cu") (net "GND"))
 (segment (start 120.220685 70.965) (end 133.75 84.494315) (width 0.2) (layer "F.Cu") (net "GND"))
 (segment (start 115.476346 91.99) (end 112.523654 91.99) (width 0.2) (layer "F.Cu") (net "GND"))
 (segment (start 111 93.513654) (end 112.523654 91.99) (width 0.2) (layer "F.Cu") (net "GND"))
 (segment (start 108 84.25) (end 112.05 88.3) (width 0.2) (layer "B.Cu") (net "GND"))
 (segment (start 109.3 104.3) (end 108.25 103.25) (width 0.2) (layer "B.Cu") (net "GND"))
 (segment (start 108.2 122.25) (end 109 122.25) (width 0.2) (layer "B.Cu") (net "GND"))
 (segment (start 109 122.25) (end 109.3 121.95) (width 0.2) (layer "B.Cu") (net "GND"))
 (segment (start 109.3 121.95) (end 109.3 104.3) (width 0.2) (layer "B.Cu") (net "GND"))
 (segment (start 109.35 85.6) (end 108 84.25) (width 0.2) (layer "B.Cu") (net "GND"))
 (segment (start 112.05 88.3) (end 115 88.3) (width 0.2) (layer "B.Cu") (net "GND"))
 (segment (start 109.35 102.2385) (end 109.35 85.6) (width 0.2) (layer "B.Cu") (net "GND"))
 (segment (start 108.3385 103.25) (end 109.35 102.2385) (width 0.2) (layer "B.Cu") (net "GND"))
 (segment (start 108.25 103.25) (end 108.3385 103.25) (width 0.2) (layer "B.Cu") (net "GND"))
 (segment (start 119.62 82.75) (end 130.25 93.38) (width 0.2) (layer "B.Cu") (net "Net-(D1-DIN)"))
 (segment (start 112.5 82.75) (end 119.62 82.75) (width 0.2) (layer "B.Cu") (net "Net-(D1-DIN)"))
 (segment (start 108 82.75) (end 112.5 82.75) (width 0.2) (layer "B.Cu") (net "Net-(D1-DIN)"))
 (segment (start 107.95 120.75) (end 107.76 120.75) (width 0.2) (layer "B.Cu") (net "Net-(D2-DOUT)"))
 (segment (start 102.8 103.25) (end 102.8 107.170101) (width 0.2) (layer "B.Cu") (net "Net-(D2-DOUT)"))
 (segment (start 107.734558 120.642331) (end 107.72582 120.66185) (width 0.2) (layer "B.Cu") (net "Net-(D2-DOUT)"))
 (segment (start 108.75 119.95) (end 107.95 120.75) (width 0.2) (layer "B.Cu") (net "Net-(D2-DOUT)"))
 (segment (start 108.75 113.120101) (end 108.75 119.95) (width 0.2) (layer "B.Cu") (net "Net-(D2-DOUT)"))
 (segment (start 102.8 107.170101) (end 108.75 113.120101) (width 0.2) (layer "B.Cu") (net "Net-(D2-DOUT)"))
 (segment (start 107.734558 120.724558) (end 107.734558 120.642331) (width 0.2) (layer "B.Cu") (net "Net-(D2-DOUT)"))
 (segment (start 107.76 120.75) (end 107.734558 120.724558) (width 0.2) (layer "B.Cu") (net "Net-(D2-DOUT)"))
 (segment (start 117.995 73.505) (end 130.25 85.76) (width 0.2) (layer "F.Cu") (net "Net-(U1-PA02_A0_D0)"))
 (segment (start 96.52 73.505) (end 117.995 73.505) (width 0.2) (layer "F.Cu") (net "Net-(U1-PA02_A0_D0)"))
 (segment (start 96.52 94.689899) (end 95.12 93.289899) (width 0.2) (layer "F.Cu") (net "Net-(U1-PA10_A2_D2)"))
 (segment (start 97.099899 75.951699) (end 97.099899 74.905) (width 0.2) (layer "F.Cu") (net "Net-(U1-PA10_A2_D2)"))
 (segment (start 133.35 88.776346) (end 131.286346 90.84) (width 0.2) (layer "F.Cu") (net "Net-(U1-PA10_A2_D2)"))
 (segment (start 97.099899 72.105) (end 97.92 72.925101) (width 0.2) (layer "F.Cu") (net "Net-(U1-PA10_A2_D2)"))
 (segment (start 95.940101 74.905) (end 95.12 74.084899) (width 0.2) (layer "F.Cu") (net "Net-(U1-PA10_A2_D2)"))
 (segment (start 133.35 84.66) (end 133.35 88.776346) (width 0.2) (layer "F.Cu") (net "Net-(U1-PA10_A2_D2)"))
 (segment (start 97.92 72.925101) (end 121.615101 72.925101) (width 0.2) (layer "F.Cu") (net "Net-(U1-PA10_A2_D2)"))
 (segment (start 96.52 111.76) (end 96.52 94.689899) (width 0.2) (layer "F.Cu") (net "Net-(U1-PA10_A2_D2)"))
 (segment (start 95.12 72.925101) (end 95.940101 72.105) (width 0.2) (layer "F.Cu") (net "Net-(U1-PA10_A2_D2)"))
 (segment (start 95.12 74.084899) (end 95.12 72.925101) (width 0.2) (layer "F.Cu") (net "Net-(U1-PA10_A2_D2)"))
 (segment (start 95.12 77.931598) (end 97.099899 75.951699) (width 0.2) (layer "F.Cu") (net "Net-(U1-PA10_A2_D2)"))
 (segment (start 131.286346 90.84) (end 130.25 90.84) (width 0.2) (layer "F.Cu") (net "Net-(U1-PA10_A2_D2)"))
 (segment (start 95.12 93.289899) (end 95.12 77.931598) (width 0.2) (layer "F.Cu") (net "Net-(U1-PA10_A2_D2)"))
 (segment (start 97.099899 74.905) (end 95.940101 74.905) (width 0.2) (layer "F.Cu") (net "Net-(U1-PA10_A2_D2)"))
 (segment (start 121.615101 72.925101) (end 133.35 84.66) (width 0.2) (layer "F.Cu") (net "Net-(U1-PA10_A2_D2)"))
 (segment (start 95.940101 72.105) (end 97.099899 72.105) (width 0.2) (layer "F.Cu") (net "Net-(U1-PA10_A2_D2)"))
 (segment (start 96.52 92.71) (end 97 92.23) (width 0.2) (layer "F.Cu") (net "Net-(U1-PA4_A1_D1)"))
 (segment (start 96.52 92.71) (end 96.52 86.343604) (width 0.2) (layer "F.Cu") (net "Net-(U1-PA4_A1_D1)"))
 (segment (start 96.52 86.343604) (end 102.563604 80.3) (width 0.2) (layer "F.Cu") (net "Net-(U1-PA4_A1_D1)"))
 (segment (start 102.563604 80.3) (end 122.25 80.3) (width 0.2) (layer "F.Cu") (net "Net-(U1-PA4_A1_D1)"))
 (segment (start 122.25 80.3) (end 130.25 88.3) (width 0.2) (layer "F.Cu") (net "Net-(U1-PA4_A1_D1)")))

